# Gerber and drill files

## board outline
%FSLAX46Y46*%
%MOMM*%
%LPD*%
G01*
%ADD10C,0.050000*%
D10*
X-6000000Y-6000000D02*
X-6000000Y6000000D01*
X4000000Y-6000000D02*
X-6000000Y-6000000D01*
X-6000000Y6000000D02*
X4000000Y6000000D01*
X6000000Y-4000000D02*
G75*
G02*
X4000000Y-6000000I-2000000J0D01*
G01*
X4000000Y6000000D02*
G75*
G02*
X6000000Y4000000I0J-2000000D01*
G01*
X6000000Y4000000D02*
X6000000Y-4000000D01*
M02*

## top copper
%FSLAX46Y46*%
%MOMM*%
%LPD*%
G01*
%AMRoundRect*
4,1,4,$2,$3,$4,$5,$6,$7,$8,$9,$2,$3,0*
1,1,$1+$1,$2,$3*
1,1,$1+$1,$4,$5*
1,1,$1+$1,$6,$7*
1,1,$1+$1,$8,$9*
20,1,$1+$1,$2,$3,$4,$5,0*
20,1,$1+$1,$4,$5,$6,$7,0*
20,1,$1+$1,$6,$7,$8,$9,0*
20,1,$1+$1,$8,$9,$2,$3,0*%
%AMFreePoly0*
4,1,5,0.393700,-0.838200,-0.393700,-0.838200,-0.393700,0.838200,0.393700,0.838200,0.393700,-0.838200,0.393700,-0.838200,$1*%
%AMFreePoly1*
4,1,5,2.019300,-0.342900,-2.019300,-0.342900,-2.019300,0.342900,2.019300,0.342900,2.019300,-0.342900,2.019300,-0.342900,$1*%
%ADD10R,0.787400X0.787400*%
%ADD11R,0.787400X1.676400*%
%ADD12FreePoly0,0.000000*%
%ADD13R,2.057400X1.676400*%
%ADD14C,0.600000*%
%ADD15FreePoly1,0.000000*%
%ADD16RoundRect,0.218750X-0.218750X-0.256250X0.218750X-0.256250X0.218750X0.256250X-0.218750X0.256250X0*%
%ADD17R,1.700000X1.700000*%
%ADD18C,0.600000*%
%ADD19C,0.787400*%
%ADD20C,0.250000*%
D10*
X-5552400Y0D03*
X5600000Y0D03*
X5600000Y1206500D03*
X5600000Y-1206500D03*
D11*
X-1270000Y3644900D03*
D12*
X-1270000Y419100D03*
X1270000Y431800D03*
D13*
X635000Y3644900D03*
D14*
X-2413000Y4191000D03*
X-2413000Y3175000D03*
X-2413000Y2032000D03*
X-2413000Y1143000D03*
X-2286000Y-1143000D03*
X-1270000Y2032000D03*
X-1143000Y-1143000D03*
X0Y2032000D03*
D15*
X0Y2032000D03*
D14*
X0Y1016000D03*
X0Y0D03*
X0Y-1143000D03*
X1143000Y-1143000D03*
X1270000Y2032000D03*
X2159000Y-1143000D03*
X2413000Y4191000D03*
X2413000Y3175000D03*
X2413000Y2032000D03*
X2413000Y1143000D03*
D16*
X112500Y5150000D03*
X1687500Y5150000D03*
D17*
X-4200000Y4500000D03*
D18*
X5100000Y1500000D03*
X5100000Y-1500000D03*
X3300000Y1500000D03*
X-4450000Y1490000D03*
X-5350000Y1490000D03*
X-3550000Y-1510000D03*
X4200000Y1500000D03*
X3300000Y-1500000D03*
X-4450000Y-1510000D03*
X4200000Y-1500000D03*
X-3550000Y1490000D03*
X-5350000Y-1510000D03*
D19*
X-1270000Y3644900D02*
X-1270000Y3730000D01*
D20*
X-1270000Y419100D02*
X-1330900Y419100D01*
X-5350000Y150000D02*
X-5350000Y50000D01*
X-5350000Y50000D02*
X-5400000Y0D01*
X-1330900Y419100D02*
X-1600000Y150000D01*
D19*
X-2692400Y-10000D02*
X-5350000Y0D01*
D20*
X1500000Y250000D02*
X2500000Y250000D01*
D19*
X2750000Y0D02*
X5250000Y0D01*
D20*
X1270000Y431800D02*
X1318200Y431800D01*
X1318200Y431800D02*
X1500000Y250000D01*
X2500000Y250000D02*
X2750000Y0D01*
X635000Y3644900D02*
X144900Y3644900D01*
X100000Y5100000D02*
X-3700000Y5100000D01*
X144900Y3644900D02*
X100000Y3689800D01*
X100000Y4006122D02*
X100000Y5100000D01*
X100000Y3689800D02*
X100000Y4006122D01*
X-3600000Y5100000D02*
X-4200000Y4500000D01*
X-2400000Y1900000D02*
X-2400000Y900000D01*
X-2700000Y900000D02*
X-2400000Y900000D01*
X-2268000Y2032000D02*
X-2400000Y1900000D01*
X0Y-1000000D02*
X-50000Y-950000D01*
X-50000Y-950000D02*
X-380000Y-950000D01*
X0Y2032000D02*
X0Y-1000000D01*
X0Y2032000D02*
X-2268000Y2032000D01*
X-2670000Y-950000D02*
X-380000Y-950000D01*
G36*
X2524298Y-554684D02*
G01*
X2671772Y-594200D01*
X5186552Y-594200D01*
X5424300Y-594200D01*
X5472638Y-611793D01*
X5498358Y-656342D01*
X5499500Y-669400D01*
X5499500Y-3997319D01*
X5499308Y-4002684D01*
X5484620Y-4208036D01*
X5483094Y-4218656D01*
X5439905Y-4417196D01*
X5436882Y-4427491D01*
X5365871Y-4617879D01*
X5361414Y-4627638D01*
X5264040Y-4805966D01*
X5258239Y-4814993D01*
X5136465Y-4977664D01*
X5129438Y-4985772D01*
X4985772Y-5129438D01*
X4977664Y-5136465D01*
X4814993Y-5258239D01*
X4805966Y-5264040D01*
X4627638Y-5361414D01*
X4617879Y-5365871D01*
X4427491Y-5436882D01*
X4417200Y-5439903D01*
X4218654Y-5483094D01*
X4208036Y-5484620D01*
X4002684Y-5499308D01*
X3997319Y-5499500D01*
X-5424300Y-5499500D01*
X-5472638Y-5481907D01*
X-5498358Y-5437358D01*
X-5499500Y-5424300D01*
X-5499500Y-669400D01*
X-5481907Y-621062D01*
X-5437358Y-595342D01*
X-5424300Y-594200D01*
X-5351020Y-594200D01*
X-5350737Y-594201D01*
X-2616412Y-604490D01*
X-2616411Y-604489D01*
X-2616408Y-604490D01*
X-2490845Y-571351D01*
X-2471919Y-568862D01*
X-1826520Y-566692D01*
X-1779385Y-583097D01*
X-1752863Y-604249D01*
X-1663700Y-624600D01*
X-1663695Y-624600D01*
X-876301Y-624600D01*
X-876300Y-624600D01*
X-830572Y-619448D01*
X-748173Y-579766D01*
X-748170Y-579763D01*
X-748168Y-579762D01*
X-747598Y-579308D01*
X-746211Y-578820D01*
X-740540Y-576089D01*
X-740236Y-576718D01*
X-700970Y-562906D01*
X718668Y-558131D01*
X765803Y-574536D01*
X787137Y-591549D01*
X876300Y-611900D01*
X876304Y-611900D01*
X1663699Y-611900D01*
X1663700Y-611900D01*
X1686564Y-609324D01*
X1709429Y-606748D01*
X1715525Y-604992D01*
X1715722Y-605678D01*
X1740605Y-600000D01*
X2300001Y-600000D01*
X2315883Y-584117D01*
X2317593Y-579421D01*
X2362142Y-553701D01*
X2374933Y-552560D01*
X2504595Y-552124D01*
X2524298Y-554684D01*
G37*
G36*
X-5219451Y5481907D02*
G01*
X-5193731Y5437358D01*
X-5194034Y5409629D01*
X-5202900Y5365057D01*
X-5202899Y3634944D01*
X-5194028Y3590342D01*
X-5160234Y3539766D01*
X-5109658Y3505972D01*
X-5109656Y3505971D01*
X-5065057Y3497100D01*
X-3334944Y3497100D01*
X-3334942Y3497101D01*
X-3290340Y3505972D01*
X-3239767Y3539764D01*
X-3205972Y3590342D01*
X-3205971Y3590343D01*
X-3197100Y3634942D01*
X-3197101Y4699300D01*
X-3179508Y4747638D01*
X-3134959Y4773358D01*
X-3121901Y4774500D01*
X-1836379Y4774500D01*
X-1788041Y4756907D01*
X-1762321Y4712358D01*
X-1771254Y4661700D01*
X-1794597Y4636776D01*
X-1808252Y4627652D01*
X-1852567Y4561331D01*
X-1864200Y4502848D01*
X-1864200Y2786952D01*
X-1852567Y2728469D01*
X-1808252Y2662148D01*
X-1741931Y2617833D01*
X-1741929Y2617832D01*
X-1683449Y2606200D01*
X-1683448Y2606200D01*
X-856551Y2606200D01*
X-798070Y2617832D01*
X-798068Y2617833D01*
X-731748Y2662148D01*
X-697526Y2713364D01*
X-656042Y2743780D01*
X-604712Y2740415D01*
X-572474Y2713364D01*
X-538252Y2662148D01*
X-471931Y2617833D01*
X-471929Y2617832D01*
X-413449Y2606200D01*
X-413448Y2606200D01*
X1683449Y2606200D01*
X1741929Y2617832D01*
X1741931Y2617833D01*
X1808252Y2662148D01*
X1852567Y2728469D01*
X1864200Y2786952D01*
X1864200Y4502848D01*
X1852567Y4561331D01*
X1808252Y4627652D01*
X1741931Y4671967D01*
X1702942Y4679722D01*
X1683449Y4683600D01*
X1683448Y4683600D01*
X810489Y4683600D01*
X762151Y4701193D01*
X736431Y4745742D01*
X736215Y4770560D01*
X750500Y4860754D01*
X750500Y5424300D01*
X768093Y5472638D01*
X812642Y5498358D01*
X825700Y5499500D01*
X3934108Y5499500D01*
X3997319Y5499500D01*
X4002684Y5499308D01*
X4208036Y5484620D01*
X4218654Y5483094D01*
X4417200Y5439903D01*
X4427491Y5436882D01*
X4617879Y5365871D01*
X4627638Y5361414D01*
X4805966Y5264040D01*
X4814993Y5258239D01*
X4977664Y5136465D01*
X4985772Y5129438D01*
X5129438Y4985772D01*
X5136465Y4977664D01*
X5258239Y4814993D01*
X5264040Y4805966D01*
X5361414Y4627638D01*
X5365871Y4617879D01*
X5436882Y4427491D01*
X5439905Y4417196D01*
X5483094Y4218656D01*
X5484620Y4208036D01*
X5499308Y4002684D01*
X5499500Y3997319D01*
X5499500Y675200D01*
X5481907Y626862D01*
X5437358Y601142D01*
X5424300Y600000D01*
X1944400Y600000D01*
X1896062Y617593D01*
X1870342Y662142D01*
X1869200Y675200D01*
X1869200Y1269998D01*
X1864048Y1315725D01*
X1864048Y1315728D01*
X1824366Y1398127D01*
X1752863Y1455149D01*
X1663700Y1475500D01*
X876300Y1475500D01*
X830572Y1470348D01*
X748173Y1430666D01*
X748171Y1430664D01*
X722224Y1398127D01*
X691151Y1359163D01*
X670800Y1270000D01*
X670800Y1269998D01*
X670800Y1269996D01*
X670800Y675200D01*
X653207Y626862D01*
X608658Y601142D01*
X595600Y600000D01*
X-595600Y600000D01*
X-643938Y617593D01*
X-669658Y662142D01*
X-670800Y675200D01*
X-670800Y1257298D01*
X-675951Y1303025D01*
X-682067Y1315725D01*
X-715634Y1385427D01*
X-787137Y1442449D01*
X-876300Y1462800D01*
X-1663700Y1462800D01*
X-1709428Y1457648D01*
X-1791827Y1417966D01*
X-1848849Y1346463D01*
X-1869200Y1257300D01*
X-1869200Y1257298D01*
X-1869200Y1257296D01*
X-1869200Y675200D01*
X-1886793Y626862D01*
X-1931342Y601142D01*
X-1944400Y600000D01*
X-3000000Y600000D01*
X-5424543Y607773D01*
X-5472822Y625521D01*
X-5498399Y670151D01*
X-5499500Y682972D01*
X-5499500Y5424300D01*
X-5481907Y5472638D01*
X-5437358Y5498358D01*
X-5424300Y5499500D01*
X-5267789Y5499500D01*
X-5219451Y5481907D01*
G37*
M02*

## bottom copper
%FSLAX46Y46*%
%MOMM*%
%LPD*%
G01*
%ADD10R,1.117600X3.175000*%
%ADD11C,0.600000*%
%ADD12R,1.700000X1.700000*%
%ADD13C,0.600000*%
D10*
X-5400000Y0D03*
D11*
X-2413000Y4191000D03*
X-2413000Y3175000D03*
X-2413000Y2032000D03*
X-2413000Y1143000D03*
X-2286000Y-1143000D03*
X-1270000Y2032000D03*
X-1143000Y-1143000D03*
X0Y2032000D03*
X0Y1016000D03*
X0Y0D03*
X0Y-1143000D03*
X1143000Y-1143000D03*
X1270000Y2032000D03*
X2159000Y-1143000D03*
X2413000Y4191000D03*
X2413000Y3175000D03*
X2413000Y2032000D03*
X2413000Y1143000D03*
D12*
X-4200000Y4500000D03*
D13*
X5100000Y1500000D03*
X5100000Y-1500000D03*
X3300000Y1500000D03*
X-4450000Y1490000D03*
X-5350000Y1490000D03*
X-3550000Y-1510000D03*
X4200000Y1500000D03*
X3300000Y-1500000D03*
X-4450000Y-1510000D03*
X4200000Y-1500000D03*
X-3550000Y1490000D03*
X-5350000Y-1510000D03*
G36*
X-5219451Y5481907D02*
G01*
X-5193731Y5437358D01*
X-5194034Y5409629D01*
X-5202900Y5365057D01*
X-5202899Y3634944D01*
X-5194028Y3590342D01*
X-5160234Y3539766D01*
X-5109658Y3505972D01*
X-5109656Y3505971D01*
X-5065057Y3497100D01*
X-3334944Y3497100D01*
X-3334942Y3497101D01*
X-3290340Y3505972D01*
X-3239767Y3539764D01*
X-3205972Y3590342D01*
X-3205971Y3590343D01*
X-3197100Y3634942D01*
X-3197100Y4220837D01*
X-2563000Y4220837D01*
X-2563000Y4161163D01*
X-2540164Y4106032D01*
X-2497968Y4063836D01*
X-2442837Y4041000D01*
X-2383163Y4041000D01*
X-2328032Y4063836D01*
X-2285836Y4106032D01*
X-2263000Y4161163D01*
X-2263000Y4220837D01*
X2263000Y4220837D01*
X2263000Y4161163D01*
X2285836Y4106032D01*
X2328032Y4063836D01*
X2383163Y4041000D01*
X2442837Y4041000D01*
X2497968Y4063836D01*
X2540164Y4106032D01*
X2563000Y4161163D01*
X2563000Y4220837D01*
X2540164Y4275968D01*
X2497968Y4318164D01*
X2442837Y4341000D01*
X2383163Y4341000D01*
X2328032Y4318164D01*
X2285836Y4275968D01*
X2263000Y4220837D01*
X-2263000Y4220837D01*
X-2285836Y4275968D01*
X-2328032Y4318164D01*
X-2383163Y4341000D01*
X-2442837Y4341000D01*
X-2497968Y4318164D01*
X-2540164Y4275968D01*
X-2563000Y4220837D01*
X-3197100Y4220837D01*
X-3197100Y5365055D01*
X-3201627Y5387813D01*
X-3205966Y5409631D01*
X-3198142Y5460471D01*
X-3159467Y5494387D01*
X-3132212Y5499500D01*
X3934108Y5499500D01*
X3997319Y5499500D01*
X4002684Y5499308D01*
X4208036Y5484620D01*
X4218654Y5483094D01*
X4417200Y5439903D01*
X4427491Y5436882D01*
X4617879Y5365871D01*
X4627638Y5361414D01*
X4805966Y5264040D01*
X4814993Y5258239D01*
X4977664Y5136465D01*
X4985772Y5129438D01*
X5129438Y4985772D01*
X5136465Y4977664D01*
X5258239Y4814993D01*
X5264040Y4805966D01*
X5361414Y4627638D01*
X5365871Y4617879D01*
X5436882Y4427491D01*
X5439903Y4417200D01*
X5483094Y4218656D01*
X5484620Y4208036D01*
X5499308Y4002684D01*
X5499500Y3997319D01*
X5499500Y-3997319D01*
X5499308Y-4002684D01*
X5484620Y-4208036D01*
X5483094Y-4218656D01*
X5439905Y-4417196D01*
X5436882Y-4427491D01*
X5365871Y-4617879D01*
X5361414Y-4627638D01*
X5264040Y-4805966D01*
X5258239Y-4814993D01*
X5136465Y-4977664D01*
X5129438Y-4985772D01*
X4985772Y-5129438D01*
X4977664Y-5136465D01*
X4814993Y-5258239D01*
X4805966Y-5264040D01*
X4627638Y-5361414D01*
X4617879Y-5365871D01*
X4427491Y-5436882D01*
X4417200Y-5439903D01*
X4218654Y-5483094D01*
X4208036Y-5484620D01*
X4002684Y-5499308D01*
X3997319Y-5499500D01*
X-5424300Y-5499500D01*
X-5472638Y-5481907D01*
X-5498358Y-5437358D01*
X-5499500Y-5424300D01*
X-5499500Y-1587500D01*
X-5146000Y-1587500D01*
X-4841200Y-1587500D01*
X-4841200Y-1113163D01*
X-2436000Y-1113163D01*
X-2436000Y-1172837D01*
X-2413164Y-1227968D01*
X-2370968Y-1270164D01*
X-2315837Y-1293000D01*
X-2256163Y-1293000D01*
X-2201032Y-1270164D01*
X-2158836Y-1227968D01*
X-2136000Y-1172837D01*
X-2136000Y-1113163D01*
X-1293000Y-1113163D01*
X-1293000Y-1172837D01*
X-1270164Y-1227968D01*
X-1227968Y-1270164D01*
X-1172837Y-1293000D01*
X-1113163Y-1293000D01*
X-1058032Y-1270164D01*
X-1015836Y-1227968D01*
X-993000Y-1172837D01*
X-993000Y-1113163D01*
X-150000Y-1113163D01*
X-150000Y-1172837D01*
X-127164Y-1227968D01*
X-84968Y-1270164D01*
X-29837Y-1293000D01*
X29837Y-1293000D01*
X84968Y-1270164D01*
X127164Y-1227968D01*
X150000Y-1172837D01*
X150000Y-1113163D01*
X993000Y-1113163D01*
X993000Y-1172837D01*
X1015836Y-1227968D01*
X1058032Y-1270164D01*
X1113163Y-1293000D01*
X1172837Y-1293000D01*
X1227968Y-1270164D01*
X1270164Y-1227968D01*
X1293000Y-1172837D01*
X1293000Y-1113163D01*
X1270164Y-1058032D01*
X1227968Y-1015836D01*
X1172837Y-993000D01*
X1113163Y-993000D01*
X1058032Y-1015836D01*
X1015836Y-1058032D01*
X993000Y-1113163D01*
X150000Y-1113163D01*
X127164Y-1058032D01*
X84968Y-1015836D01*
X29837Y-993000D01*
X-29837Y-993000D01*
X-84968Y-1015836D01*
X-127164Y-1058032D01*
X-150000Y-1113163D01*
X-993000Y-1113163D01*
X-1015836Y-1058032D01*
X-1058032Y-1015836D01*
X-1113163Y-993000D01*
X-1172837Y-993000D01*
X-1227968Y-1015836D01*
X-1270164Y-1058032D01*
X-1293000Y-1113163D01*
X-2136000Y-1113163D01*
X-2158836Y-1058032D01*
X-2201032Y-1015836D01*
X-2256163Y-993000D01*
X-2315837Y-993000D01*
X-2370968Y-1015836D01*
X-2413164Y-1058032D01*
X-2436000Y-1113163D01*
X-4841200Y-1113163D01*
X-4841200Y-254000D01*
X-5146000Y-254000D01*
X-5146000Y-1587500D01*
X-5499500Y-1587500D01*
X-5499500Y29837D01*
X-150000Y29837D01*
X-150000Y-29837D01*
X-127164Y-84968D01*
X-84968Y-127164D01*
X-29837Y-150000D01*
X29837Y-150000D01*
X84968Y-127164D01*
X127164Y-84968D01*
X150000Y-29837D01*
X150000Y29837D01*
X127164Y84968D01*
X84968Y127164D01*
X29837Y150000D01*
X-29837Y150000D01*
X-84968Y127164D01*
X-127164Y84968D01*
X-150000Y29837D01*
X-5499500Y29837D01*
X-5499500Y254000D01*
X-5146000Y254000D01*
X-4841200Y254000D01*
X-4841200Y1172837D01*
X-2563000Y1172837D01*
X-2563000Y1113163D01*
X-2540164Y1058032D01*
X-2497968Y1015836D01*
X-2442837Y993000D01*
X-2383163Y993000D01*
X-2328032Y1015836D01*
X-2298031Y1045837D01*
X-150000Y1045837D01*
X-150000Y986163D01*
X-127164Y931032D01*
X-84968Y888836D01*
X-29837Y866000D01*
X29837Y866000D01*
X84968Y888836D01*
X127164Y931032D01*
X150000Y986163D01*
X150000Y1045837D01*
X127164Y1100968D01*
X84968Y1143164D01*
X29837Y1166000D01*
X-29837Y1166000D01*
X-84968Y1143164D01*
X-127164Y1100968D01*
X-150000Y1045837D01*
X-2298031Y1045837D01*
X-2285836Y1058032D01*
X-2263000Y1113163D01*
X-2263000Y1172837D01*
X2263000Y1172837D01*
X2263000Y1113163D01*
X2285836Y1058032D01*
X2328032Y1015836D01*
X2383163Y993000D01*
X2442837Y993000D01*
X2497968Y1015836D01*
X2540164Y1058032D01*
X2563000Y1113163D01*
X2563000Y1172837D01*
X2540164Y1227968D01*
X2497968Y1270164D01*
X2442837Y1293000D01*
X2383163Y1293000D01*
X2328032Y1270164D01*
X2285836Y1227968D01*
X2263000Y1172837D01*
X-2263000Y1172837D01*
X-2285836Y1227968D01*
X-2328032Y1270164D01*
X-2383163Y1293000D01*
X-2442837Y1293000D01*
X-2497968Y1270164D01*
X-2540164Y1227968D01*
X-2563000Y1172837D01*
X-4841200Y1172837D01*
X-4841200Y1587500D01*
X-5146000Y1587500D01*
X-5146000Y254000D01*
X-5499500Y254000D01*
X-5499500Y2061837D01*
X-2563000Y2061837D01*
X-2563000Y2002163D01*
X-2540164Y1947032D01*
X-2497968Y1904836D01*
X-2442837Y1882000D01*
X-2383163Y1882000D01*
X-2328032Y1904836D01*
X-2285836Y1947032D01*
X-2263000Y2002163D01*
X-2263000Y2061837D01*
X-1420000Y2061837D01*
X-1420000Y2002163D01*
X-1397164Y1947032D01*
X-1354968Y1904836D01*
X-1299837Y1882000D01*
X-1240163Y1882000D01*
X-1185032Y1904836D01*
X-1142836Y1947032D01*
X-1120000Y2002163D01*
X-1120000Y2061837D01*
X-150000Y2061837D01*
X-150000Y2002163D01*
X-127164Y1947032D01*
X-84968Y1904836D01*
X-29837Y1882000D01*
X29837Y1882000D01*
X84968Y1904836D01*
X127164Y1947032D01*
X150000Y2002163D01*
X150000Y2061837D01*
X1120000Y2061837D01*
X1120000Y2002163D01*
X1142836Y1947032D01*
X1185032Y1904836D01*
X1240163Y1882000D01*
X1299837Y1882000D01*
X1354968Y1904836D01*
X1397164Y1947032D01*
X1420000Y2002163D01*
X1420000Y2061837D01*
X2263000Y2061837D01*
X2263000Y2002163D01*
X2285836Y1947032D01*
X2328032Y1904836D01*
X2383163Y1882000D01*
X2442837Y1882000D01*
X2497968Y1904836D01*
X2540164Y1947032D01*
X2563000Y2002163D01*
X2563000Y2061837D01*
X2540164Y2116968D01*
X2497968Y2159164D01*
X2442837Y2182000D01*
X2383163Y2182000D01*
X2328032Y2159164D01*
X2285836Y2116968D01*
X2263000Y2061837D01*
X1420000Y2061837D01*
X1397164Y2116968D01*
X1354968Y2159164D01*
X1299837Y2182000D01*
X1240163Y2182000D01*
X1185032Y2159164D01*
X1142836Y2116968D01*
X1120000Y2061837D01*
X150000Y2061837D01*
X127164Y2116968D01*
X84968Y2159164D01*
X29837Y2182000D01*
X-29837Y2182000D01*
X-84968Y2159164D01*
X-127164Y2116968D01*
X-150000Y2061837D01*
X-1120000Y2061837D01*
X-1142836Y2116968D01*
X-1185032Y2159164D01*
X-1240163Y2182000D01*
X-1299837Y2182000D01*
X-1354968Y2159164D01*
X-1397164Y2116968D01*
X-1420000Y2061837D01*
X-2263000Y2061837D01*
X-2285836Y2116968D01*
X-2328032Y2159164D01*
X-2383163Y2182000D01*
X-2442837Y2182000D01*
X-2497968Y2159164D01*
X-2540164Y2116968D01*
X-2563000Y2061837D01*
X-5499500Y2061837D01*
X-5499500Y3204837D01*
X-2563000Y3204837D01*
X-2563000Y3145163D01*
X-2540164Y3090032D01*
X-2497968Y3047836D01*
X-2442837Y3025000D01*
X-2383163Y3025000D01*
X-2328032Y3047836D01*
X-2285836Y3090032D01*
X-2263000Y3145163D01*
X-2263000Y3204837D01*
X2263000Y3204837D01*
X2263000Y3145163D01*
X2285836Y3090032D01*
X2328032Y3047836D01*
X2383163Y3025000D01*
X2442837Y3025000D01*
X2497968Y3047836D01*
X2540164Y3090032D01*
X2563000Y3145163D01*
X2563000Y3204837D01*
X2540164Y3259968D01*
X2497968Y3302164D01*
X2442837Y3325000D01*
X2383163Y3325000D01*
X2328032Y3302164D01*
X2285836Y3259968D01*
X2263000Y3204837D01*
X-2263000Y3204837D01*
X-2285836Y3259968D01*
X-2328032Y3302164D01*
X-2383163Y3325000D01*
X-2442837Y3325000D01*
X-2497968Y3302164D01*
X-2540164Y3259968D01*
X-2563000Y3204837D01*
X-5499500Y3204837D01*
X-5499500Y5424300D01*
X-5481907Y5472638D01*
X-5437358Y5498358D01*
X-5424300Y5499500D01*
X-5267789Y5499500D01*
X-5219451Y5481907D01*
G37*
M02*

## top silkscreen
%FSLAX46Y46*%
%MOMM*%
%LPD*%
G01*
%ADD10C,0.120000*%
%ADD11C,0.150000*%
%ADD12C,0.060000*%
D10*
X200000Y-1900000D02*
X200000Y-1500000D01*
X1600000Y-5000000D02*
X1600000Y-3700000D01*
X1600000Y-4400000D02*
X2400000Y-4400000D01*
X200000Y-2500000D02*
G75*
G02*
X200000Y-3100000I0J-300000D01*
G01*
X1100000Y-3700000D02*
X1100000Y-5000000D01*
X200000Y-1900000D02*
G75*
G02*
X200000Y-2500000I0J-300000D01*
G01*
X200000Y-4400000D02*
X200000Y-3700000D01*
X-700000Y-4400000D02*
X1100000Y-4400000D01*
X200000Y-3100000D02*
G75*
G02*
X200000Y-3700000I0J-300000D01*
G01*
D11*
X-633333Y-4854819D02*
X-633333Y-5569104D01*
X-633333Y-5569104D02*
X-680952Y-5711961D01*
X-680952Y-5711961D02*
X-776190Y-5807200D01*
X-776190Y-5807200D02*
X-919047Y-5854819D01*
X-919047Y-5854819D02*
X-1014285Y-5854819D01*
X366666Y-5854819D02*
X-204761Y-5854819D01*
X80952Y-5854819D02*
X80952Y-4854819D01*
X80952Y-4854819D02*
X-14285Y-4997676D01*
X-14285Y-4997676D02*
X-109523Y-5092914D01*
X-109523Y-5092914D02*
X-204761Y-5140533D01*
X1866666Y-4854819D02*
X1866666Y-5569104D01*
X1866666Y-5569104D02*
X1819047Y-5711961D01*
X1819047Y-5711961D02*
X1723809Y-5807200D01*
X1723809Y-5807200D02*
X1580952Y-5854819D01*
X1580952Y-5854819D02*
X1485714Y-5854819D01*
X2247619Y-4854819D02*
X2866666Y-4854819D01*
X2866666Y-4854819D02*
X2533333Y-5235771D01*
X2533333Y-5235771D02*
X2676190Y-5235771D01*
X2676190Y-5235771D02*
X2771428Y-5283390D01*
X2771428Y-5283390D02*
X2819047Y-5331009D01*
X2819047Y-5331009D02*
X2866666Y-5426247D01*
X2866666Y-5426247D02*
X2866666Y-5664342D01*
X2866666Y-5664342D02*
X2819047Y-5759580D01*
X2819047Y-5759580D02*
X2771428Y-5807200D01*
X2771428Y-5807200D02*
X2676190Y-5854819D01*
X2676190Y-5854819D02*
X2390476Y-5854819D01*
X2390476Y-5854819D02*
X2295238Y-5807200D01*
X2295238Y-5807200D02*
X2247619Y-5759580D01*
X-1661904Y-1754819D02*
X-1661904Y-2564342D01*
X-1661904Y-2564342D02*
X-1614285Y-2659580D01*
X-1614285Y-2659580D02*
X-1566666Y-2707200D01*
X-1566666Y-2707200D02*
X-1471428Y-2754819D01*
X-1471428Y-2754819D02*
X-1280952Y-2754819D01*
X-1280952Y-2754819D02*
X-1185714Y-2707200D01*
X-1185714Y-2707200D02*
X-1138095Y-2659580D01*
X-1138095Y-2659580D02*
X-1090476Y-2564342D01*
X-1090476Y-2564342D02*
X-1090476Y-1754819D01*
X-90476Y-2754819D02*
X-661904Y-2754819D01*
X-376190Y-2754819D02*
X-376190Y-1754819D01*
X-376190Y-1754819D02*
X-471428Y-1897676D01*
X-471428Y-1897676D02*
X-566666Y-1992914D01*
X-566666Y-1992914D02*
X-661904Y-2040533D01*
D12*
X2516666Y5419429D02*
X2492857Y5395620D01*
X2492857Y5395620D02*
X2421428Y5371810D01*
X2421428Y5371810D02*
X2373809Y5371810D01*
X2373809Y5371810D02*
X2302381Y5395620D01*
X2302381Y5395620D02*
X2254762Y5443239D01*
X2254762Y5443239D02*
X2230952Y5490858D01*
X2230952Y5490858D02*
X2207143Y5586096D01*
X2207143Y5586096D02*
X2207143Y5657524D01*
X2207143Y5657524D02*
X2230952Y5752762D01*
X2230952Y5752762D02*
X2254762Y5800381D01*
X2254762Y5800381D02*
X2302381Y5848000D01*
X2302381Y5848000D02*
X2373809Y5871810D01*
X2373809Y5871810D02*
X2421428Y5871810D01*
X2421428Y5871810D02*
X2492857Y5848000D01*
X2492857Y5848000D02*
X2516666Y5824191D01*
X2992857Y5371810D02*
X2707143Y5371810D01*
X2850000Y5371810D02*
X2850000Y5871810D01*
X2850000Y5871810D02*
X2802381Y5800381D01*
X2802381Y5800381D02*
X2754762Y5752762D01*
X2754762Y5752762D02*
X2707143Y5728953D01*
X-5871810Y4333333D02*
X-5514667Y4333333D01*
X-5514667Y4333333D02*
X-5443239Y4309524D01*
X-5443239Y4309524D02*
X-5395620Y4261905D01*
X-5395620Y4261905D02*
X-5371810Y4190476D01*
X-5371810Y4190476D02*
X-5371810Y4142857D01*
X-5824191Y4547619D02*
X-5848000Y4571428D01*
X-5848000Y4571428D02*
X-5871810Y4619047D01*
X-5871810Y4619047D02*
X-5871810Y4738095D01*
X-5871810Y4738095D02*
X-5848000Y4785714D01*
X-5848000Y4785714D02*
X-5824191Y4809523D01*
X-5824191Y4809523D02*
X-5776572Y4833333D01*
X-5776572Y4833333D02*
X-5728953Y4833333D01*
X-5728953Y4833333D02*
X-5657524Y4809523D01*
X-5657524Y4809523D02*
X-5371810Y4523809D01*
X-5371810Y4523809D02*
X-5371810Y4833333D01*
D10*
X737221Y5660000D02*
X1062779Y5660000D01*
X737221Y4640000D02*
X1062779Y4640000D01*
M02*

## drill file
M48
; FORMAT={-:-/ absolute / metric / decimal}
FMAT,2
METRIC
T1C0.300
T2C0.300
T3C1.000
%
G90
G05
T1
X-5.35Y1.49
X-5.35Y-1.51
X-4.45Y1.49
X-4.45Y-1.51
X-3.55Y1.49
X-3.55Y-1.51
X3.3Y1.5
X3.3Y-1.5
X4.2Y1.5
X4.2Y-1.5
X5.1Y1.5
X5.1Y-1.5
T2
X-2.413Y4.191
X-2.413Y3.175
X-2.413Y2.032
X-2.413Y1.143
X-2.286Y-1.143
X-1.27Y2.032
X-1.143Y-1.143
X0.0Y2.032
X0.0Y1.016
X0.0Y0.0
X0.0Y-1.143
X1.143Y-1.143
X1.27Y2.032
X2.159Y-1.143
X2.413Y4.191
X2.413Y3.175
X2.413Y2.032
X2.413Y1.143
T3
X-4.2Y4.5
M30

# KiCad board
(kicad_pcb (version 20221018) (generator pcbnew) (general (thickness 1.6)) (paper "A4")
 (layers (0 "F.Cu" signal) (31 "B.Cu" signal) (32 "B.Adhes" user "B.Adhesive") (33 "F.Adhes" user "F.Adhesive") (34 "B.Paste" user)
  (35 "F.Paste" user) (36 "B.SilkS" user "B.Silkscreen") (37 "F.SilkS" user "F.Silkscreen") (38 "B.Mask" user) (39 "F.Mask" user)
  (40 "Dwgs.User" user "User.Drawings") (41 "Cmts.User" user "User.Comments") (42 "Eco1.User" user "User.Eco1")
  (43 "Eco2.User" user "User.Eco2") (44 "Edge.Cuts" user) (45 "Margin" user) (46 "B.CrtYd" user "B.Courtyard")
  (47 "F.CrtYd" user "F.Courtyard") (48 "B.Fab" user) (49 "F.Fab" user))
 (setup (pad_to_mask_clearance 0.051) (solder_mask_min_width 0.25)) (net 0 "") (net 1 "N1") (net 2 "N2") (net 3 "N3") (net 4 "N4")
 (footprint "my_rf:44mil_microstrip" (layer "F.Cu") (at -5.4 0)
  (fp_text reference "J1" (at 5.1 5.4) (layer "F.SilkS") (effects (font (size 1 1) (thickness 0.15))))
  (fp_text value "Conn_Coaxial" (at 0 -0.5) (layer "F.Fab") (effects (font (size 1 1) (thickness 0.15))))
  (pad "1" smd rect (at -0.1524 0) (size 0.7874 0.7874) (layers "F.Cu" "F.Mask") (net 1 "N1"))
  (pad "2" smd rect (at 0 0) (size 1.1176 3.175) (layers "B.Cu" "B.Mask") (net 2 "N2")))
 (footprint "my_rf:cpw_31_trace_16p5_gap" (layer "F.Cu") (at 5.6 0)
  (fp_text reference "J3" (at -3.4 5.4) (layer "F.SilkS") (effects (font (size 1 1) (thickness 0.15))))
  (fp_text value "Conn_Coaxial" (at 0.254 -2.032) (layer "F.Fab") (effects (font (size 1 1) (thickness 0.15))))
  (pad "1" smd rect (at 0 0) (size 0.7874 0.7874) (layers "F.Cu" "F.Mask") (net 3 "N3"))
  (pad "2" smd rect (at 0 -1.2065) (size 0.7874 0.7874) (layers "F.Cu") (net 2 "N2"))
  (pad "2" smd rect (at 0 1.2065) (size 0.7874 0.7874) (layers "F.Cu") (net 2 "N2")))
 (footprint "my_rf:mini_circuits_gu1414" (layer "F.Cu") (at 0 -2.032)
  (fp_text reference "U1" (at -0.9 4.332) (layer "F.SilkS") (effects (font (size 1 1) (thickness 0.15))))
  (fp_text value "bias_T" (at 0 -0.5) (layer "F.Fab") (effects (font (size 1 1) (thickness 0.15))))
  (pad "" smd rect (at -1.27 -1.6129) (size 0.7874 1.6764) (layers "F.Cu" "F.Paste"))
  (pad "1" smd custom (at -1.27 1.6129) (size 0.7874 1.6764) (layers "F.Cu") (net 1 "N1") (zone_connect 0) (thermal_bridge_angle 45)
   (options (clearance outline) (anchor rect)) (primitives))
  (pad "2" smd custom (at 1.27 1.6002) (size 0.7874 1.6764) (layers "F.Cu") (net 3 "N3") (zone_connect 0) (thermal_bridge_angle 45)
   (options (clearance outline) (anchor rect)) (primitives))
  (pad "3" smd rect (at 0.635 -1.6129) (size 2.0574 1.6764) (layers "F.Cu") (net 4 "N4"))
  (pad "4" thru_hole circle (at -2.413 -2.159) (size 0.6 0.6) (drill 0.3) (layers "*.Cu") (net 2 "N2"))
  (pad "4" thru_hole circle (at -2.413 -1.143) (size 0.6 0.6) (drill 0.3) (layers "*.Cu") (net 2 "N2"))
  (pad "4" thru_hole circle (at -2.413 0) (size 0.6 0.6) (drill 0.3) (layers "*.Cu") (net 2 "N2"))
  (pad "4" thru_hole circle (at -2.413 0.889) (size 0.6 0.6) (drill 0.3) (layers "*.Cu") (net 2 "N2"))
  (pad "4" thru_hole circle (at -2.286 3.175) (size 0.6 0.6) (drill 0.3) (layers "*.Cu") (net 2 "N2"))
  (pad "4" thru_hole circle (at -1.27 0) (size 0.6 0.6) (drill 0.3) (layers "*.Cu") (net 2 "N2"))
  (pad "4" thru_hole circle (at -1.143 3.175) (size 0.6 0.6) (drill 0.3) (layers "*.Cu") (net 2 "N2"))
  (pad "4" thru_hole circle (at 0 0) (size 0.6 0.6) (drill 0.3) (layers "*.Cu") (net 2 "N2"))
  (pad "4" smd custom (at 0 0) (size 4.0386 0.6858) (layers "F.Cu") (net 2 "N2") (zone_connect 2) (thermal_bridge_angle 45)
   (options (clearance outline) (anchor rect)) (primitives))
  (pad "4" thru_hole circle (at 0 1.016) (size 0.6 0.6) (drill 0.3) (layers "*.Cu") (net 2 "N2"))
  (pad "4" thru_hole circle (at 0 2.032) (size 0.6 0.6) (drill 0.3) (layers "*.Cu") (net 2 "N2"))
  (pad "4" thru_hole circle (at 0 3.175) (size 0.6 0.6) (drill 0.3) (layers "*.Cu") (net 2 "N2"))
  (pad "4" thru_hole circle (at 1.143 3.175) (size 0.6 0.6) (drill 0.3) (layers "*.Cu") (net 2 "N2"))
  (pad "4" thru_hole circle (at 1.27 0) (size 0.6 0.6) (drill 0.3) (layers "*.Cu") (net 2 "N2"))
  (pad "4" thru_hole circle (at 2.159 3.175) (size 0.6 0.6) (drill 0.3) (layers "*.Cu") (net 2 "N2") (zone_connect 2))
  (pad "4" thru_hole circle (at 2.413 -2.159) (size 0.6 0.6) (drill 0.3) (layers "*.Cu") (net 2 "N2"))
  (pad "4" thru_hole circle (at 2.413 -1.143) (size 0.6 0.6) (drill 0.3) (layers "*.Cu") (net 2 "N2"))
  (pad "4" thru_hole circle (at 2.413 0) (size 0.6 0.6) (drill 0.3) (layers "*.Cu") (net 2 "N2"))
  (pad "4" thru_hole circle (at 2.413 0.889) (size 0.6 0.6) (drill 0.3) (layers "*.Cu") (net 2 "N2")))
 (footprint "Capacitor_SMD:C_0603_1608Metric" (layer "F.Cu") (at 0.9 -5.15)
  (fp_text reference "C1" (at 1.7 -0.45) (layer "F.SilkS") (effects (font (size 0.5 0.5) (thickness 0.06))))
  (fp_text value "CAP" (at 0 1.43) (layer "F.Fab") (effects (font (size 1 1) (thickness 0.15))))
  (fp_line (start -0.162779 -0.51) (end 0.162779 -0.51) (stroke (width 0.12) (type solid)) (layer "F.SilkS"))
  (fp_line (start -0.162779 0.51) (end 0.162779 0.51) (stroke (width 0.12) (type solid)) (layer "F.SilkS"))
  (pad "1" smd roundrect (at -0.7875 0) (size 0.875 0.95) (layers "F.Cu" "F.Paste" "F.Mask") (roundrect_rratio 0.25) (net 4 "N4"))
  (pad "2" smd roundrect (at 0.7875 0) (size 0.875 0.95) (layers "F.Cu" "F.Paste" "F.Mask") (roundrect_rratio 0.25) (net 2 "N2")))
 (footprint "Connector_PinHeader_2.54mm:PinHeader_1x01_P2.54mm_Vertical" (layer "B.Cu") (at -4.2 -4.5)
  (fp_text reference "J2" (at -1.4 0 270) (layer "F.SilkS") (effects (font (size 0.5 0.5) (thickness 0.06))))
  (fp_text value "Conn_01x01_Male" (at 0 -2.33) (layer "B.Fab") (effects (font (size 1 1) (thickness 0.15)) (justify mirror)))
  (pad "1" thru_hole rect (at 0 0) (size 1.7 1.7) (drill 1) (layers "*.Cu" "*.Mask") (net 4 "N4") (clearance 0.1524)))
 (gr_line (start 0.2 1.9) (end 0.2 1.5) (stroke (width 0.12) (type solid)) (layer "F.SilkS"))
 (gr_line (start 1.6 5) (end 1.6 3.7) (stroke (width 0.12) (type solid)) (layer "F.SilkS"))
 (gr_line (start 1.6 4.4) (end 2.4 4.4) (stroke (width 0.12) (type solid)) (layer "F.SilkS"))
 (gr_arc (start 0.2 2.5) (mid 0.5 2.8) (end 0.2 3.1) (stroke (width 0.12) (type solid)) (layer "F.SilkS"))
 (gr_line (start 1.1 3.7) (end 1.1 5) (stroke (width 0.12) (type solid)) (layer "F.SilkS"))
 (gr_arc (start 0.2 1.9) (mid 0.5 2.2) (end 0.2 2.5) (stroke (width 0.12) (type solid)) (layer "F.SilkS"))
 (gr_line (start 0.2 4.4) (end 0.2 3.7) (stroke (width 0.12) (type solid)) (layer "F.SilkS"))
 (gr_line (start -0.7 4.4) (end 1.1 4.4) (stroke (width 0.12) (type solid)) (layer "F.SilkS"))
 (gr_arc (start 0.2 3.1) (mid 0.5 3.4) (end 0.2 3.7) (stroke (width 0.12) (type solid)) (layer "F.SilkS"))
 (gr_line (start -6 6) (end -6 -6) (stroke (width 0.05) (type solid)) (layer "Edge.Cuts"))
 (gr_line (start 4 6) (end -6 6) (stroke (width 0.05) (type solid)) (layer "Edge.Cuts"))
 (gr_line (start -6 -6) (end 4 -6) (stroke (width 0.05) (type solid)) (layer "Edge.Cuts"))
 (gr_arc (start 6 4) (mid 5.414214 5.414214) (end 4 6) (stroke (width 0.05) (type solid)) (layer "Edge.Cuts"))
 (gr_arc (start 4 -6) (mid 5.414214 -5.414214) (end 6 -4) (stroke (width 0.05) (type solid)) (layer "Edge.Cuts"))
 (gr_line (start 6 -4) (end 6 4) (stroke (width 0.05) (type solid)) (layer "Edge.Cuts"))
 (segment (start -1.27 -3.6449) (end -1.27 -3.73) (width 0.7874) (layer "F.Cu") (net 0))
 (segment (start -1.27 -0.4191) (end -1.3309 -0.4191) (width 0.25) (layer "F.Cu") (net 1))
 (segment (start -5.35 -0.15) (end -5.35 -0.05) (width 0.25) (layer "F.Cu") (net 1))
 (segment (start -5.35 -0.05) (end -5.4 0) (width 0.25) (layer "F.Cu") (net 1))
 (segment (start -1.3309 -0.4191) (end -1.6 -0.15) (width 0.25) (layer "F.Cu") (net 1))
 (segment (start -2.6924 0.01) (end -5.35 0) (width 0.7874) (layer "F.Cu") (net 1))
 (segment (start 1.5 -0.25) (end 2.5 -0.25) (width 0.25) (layer "F.Cu") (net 3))
 (segment (start 2.75 0) (end 5.25 0) (width 0.7874) (layer "F.Cu") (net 3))
 (segment (start 1.27 -0.4318) (end 1.3182 -0.4318) (width 0.25) (layer "F.Cu") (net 3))
 (segment (start 1.3182 -0.4318) (end 1.5 -0.25) (width 0.25) (layer "F.Cu") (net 3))
 (segment (start 2.5 -0.25) (end 2.75 0) (width 0.25) (layer "F.Cu") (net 3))
 (segment (start 0.635 -3.6449) (end 0.1449 -3.6449) (width 0.25) (layer "F.Cu") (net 4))
 (segment (start 0.1 -5.1) (end -3.7 -5.1) (width 0.25) (layer "F.Cu") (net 4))
 (segment (start 0.1449 -3.6449) (end 0.1 -3.6898) (width 0.25) (layer "F.Cu") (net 4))
 (segment (start 0.1 -4.006122) (end 0.1 -5.1) (width 0.25) (layer "F.Cu") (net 4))
 (segment (start 0.1 -3.6898) (end 0.1 -4.006122) (width 0.25) (layer "F.Cu") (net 4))
 (segment (start -3.6 -5.1) (end -4.2 -4.5) (width 0.25) (layer "F.Cu") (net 4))
 (segment (start -2.4 -1.9) (end -2.4 -0.9) (width 0.25) (layer "F.Cu") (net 2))
 (segment (start -2.7 -0.9) (end -2.4 -0.9) (width 0.25) (layer "F.Cu") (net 2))
 (segment (start -2.268 -2.032) (end -2.4 -1.9) (width 0.25) (layer "F.Cu") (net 2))
 (segment (start 0 1) (end -0.05 0.95) (width 0.25) (layer "F.Cu") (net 2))
 (segment (start -0.05 0.95) (end -0.38 0.95) (width 0.25) (layer "F.Cu") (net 2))
 (segment (start 0 -2.032) (end 0 1) (width 0.25) (layer "F.Cu") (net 2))
 (segment (start 0 -2.032) (end -2.268 -2.032) (width 0.25) (layer "F.Cu") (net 2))
 (segment (start -2.67 0.95) (end -0.38 0.95) (width 0.25) (layer "F.Cu") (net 2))
 (via (at 5.1 -1.5) (size 0.6) (drill 0.3) (layers "F.Cu" "B.Cu") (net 2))
 (via (at 5.1 1.5) (size 0.6) (drill 0.3) (layers "F.Cu" "B.Cu") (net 2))
 (via (at 3.3 -1.5) (size 0.6) (drill 0.3) (layers "F.Cu" "B.Cu") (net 2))
 (via (at -4.45 -1.49) (size 0.6) (drill 0.3) (layers "F.Cu" "B.Cu") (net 2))
 (via (at -5.35 -1.49) (size 0.6) (drill 0.3) (layers "F.Cu" "B.Cu") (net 2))
 (via (at -3.55 1.51) (size 0.6) (drill 0.3) (layers "F.Cu" "B.Cu") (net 2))
 (via (at 4.2 -1.5) (size 0.6) (drill 0.3) (layers "F.Cu" "B.Cu") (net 2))
 (via (at 3.3 1.5) (size 0.6) (drill 0.3) (layers "F.Cu" "B.Cu") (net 2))
 (via (at -4.45 1.51) (size 0.6) (drill 0.3) (layers "F.Cu" "B.Cu") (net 2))
 (via (at 4.2 1.5) (size 0.6) (drill 0.3) (layers "F.Cu" "B.Cu") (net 2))
 (via (at -3.55 -1.49) (size 0.6) (drill 0.3) (layers "F.Cu" "B.Cu") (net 2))
 (via (at -5.35 1.51) (size 0.6) (drill 0.3) (layers "F.Cu" "B.Cu") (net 2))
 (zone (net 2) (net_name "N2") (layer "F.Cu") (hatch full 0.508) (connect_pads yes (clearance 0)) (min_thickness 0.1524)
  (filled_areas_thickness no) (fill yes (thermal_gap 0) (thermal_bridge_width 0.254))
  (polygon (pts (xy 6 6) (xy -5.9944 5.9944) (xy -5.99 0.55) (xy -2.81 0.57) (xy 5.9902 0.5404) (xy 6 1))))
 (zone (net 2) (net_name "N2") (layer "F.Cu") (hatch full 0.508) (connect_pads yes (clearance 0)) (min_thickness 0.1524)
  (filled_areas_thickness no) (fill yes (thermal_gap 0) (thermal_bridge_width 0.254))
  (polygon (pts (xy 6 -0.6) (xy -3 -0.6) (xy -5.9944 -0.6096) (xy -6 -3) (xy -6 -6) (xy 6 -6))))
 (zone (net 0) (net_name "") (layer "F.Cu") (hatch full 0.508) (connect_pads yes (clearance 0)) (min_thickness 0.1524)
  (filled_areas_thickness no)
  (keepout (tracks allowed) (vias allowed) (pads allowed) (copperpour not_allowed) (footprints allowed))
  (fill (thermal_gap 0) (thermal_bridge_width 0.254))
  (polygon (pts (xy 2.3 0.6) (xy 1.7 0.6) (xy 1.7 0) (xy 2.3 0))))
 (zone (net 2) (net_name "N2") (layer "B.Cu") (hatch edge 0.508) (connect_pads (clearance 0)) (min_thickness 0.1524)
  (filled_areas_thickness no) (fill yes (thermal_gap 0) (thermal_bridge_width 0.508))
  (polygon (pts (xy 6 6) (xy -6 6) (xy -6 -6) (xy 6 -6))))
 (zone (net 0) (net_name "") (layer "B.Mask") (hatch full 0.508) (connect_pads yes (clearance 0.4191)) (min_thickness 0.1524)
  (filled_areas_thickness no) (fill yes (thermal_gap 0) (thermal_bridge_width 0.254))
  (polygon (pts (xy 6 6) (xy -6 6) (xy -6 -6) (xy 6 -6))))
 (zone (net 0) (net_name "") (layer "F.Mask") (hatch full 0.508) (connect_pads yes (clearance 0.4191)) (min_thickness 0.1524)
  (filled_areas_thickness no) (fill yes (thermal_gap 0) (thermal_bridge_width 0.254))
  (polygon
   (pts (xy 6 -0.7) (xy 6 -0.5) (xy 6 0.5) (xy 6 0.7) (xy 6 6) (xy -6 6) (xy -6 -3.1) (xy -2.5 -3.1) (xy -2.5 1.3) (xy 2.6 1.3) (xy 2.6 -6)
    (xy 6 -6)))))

